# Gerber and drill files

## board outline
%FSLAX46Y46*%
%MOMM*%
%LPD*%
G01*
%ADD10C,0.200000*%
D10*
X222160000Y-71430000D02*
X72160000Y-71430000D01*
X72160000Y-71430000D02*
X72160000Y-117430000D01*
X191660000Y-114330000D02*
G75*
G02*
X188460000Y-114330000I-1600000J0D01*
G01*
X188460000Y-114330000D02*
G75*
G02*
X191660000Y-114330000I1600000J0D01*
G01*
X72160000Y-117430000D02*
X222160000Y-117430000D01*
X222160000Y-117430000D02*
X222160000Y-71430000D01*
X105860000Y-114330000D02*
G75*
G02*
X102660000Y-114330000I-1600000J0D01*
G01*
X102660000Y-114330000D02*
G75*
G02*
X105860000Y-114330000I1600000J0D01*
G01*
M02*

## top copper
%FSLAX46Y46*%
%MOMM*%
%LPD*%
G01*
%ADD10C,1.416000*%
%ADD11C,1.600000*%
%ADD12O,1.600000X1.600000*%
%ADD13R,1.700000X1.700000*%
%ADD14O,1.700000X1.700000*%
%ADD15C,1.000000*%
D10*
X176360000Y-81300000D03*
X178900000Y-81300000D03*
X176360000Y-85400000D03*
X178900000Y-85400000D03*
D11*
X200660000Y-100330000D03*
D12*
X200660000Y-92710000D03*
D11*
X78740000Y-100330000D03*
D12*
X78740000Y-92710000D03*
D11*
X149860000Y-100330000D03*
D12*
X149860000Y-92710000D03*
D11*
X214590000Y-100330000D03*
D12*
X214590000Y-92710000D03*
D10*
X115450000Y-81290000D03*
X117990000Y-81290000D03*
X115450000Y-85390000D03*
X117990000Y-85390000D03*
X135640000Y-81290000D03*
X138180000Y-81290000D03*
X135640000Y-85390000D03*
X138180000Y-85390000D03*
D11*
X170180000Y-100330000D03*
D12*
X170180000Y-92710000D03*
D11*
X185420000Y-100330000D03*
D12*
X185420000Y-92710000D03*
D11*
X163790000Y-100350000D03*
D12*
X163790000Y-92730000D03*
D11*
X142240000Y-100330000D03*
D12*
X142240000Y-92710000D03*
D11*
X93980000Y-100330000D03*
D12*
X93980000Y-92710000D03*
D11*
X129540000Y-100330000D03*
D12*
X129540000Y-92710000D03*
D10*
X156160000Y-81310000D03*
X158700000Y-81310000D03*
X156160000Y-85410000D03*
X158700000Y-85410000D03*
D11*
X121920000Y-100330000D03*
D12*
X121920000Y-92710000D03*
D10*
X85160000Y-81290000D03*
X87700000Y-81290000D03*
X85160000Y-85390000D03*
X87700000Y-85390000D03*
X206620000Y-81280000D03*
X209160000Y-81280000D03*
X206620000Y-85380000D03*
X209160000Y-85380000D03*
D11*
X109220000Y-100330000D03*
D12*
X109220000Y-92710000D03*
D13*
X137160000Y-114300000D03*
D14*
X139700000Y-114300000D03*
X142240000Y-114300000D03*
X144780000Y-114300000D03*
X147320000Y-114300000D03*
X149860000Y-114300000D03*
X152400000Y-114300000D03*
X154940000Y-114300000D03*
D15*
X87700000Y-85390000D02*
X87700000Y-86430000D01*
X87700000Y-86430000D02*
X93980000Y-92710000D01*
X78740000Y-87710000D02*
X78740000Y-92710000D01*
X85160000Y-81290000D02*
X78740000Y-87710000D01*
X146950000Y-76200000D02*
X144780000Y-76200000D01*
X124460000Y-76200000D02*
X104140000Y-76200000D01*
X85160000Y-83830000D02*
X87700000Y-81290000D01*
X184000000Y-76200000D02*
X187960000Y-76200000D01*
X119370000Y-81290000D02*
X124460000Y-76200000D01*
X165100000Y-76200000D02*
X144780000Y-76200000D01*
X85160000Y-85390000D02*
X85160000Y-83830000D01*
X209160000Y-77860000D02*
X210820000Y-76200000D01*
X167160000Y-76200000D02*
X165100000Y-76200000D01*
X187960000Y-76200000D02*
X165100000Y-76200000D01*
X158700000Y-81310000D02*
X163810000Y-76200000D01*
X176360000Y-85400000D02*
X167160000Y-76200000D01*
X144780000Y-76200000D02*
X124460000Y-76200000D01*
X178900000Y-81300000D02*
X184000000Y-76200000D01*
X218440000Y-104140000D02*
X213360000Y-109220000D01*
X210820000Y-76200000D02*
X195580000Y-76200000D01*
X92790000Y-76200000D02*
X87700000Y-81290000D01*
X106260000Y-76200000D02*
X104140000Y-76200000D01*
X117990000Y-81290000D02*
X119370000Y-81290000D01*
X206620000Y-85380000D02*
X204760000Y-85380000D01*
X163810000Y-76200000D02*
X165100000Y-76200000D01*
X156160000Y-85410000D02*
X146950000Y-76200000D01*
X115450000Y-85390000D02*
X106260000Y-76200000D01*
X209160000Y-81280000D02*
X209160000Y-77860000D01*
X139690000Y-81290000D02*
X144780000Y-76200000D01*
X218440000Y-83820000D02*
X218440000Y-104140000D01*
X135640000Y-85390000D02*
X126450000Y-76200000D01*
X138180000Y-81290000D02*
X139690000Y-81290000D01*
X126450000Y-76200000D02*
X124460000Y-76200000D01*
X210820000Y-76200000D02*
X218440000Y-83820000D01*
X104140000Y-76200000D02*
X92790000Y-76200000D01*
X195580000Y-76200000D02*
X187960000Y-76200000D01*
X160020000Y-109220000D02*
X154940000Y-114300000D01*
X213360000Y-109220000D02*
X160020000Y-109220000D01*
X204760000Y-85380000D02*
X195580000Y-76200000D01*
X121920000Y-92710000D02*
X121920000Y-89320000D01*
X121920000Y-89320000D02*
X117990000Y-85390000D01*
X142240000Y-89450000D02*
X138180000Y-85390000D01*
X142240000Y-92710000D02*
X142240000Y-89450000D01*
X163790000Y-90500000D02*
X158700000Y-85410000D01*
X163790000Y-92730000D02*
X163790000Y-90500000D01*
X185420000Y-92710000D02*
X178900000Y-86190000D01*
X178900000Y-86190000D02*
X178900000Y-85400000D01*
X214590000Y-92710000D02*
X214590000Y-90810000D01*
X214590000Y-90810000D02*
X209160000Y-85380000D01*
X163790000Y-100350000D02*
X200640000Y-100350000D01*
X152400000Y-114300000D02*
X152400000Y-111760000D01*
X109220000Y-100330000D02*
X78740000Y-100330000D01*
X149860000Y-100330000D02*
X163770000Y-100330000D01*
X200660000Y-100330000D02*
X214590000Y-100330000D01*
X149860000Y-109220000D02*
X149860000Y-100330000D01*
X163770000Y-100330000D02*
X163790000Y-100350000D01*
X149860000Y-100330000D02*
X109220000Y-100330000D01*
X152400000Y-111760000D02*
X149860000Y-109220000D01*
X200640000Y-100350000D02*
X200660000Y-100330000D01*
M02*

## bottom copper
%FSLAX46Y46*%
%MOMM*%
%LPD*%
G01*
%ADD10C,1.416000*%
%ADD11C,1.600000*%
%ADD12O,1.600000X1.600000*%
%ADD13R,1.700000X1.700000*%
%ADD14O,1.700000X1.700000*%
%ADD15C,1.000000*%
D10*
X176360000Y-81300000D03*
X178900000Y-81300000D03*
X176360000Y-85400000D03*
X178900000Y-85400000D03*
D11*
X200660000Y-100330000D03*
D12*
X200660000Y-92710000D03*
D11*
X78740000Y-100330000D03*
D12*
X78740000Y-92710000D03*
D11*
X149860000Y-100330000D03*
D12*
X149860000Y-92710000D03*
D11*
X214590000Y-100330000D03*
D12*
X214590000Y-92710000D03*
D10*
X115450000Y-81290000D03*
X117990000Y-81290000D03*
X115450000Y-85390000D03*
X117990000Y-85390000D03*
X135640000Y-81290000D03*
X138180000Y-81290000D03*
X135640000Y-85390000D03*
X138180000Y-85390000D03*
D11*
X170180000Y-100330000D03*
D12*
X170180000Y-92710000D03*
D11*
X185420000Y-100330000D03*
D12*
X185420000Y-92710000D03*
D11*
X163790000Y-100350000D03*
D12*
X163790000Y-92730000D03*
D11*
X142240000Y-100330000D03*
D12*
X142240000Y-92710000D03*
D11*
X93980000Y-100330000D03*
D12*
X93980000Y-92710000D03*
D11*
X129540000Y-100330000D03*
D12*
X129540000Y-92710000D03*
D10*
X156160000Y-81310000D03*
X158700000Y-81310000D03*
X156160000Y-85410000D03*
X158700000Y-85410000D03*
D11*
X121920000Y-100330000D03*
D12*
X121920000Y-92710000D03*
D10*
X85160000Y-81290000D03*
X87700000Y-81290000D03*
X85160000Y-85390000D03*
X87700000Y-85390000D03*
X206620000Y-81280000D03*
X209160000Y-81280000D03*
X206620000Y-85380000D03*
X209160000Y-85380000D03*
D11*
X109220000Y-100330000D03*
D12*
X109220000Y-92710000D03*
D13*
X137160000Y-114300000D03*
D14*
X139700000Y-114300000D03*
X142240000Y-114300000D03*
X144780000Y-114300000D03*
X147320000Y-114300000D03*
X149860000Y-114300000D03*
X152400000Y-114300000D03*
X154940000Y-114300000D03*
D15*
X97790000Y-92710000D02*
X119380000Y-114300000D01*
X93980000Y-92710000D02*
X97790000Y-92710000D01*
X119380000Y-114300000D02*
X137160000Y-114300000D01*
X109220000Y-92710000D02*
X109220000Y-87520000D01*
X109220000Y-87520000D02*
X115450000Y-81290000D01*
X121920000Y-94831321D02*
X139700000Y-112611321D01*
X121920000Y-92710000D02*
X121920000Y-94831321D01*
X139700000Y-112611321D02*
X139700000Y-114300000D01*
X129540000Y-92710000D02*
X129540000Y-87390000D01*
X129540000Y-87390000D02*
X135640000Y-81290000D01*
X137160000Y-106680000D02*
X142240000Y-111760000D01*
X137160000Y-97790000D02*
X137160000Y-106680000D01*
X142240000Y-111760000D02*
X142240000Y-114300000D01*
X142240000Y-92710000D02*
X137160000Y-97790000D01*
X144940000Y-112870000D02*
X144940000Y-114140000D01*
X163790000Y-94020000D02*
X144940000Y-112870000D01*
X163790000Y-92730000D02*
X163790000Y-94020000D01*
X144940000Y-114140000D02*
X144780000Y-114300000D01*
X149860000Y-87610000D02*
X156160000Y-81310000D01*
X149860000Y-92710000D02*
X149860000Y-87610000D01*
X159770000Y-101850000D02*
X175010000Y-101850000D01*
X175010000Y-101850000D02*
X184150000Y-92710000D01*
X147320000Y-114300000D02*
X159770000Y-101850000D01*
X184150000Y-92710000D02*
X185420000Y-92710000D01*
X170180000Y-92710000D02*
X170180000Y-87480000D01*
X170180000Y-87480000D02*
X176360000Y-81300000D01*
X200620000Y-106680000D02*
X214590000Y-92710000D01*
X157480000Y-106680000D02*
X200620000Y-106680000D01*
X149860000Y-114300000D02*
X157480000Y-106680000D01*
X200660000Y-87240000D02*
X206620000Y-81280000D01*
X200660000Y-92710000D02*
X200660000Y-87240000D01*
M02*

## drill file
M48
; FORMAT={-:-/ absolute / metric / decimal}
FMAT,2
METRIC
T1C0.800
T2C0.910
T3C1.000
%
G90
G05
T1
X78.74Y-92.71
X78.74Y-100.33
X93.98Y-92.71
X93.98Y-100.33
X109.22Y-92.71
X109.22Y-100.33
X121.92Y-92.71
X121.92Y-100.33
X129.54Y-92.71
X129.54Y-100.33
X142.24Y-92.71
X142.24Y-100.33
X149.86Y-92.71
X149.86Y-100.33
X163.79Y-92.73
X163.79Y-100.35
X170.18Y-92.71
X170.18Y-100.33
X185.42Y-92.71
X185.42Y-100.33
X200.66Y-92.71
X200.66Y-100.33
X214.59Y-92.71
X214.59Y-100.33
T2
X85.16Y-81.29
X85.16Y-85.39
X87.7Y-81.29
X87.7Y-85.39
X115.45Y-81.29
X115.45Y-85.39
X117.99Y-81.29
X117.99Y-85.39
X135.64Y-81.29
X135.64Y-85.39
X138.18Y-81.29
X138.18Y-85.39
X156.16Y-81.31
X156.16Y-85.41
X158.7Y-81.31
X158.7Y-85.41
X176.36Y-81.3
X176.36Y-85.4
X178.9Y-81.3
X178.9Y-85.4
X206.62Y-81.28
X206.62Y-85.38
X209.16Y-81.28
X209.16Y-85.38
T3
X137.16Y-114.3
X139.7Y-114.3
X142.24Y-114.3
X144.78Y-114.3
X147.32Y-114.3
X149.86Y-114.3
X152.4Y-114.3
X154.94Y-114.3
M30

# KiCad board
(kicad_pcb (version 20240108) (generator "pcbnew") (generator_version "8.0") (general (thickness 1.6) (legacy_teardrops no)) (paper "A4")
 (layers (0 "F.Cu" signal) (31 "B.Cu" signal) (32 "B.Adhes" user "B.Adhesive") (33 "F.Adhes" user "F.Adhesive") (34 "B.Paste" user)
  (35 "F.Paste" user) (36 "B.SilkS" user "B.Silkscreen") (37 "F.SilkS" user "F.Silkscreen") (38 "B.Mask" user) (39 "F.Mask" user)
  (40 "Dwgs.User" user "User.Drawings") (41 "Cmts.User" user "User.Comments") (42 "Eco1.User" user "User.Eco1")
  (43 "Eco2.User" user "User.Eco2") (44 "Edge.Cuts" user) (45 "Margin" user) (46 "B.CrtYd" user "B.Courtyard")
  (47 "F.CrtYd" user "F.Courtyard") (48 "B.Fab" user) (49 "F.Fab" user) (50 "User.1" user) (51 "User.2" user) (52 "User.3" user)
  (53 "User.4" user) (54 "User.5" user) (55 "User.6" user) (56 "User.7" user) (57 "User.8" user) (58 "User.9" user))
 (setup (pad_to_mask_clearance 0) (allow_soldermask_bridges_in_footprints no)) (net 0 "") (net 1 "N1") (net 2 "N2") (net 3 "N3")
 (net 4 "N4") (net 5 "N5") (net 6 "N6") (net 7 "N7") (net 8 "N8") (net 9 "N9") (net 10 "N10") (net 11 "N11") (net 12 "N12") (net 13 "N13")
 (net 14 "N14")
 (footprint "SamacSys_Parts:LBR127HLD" (layer "F.Cu") (at 176.36 81.3 90)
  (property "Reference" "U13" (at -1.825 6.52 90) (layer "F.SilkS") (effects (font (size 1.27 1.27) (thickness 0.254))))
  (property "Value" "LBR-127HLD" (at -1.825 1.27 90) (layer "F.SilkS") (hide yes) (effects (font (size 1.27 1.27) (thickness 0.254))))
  (pad "1" thru_hole circle (at 0 0 90) (size 1.416 1.416) (drill 0.91) (layers "*.Cu" "*.Mask") (remove_unused_layers no) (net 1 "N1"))
  (pad "2" thru_hole circle (at 0 2.54 90) (size 1.416 1.416) (drill 0.91) (layers "*.Cu" "*.Mask") (remove_unused_layers no) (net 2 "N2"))
  (pad "3" thru_hole circle (at -4.1 0 90) (size 1.416 1.416) (drill 0.91) (layers "*.Cu" "*.Mask") (remove_unused_layers no) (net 2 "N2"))
  (pad "4" thru_hole circle (at -4.1 2.54 90) (size 1.416 1.416) (drill 0.91) (layers "*.Cu" "*.Mask") (remove_unused_layers no)
   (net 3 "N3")))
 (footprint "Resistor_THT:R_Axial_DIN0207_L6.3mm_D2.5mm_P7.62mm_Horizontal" (layer "F.Cu") (at 200.66 100.33 90)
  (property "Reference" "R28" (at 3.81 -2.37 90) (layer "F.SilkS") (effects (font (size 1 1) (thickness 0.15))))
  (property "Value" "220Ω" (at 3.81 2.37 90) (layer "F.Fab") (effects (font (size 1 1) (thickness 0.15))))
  (pad "1" thru_hole circle (at 0 0 90) (size 1.6 1.6) (drill 0.8) (layers "*.Cu" "*.Mask") (remove_unused_layers no) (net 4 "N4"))
  (pad "2" thru_hole oval (at 7.62 0 90) (size 1.6 1.6) (drill 0.8) (layers "*.Cu" "*.Mask") (remove_unused_layers no) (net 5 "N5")))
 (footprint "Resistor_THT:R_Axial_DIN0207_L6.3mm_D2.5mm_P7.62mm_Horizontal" (layer "F.Cu") (at 78.74 100.33 90)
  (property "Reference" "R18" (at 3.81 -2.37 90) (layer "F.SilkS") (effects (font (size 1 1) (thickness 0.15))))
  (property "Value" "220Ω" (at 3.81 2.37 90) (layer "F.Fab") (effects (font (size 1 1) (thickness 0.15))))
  (pad "1" thru_hole circle (at 0 0 90) (size 1.6 1.6) (drill 0.8) (layers "*.Cu" "*.Mask") (remove_unused_layers no) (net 4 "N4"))
  (pad "2" thru_hole oval (at 7.62 0 90) (size 1.6 1.6) (drill 0.8) (layers "*.Cu" "*.Mask") (remove_unused_layers no) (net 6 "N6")))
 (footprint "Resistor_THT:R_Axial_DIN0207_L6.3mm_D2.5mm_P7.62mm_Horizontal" (layer "F.Cu") (at 149.86 100.33 90)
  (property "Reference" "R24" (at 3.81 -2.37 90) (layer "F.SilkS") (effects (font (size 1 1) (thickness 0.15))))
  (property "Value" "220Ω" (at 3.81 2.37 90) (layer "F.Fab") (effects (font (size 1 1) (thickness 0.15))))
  (pad "1" thru_hole circle (at 0 0 90) (size 1.6 1.6) (drill 0.8) (layers "*.Cu" "*.Mask") (remove_unused_layers no) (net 4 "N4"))
  (pad "2" thru_hole oval (at 7.62 0 90) (size 1.6 1.6) (drill 0.8) (layers "*.Cu" "*.Mask") (remove_unused_layers no) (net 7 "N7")))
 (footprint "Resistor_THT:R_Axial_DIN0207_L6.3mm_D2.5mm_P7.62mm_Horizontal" (layer "F.Cu") (at 214.59 100.33 90)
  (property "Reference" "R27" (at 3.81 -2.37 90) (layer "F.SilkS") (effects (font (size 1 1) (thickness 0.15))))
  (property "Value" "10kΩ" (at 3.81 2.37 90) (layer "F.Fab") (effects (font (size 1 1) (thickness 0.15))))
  (pad "1" thru_hole circle (at 0 0 90) (size 1.6 1.6) (drill 0.8) (layers "*.Cu" "*.Mask") (remove_unused_layers no) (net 4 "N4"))
  (pad "2" thru_hole oval (at 7.62 0 90) (size 1.6 1.6) (drill 0.8) (layers "*.Cu" "*.Mask") (remove_unused_layers no) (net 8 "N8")))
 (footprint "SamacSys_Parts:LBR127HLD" (layer "F.Cu") (at 115.45 81.29 90)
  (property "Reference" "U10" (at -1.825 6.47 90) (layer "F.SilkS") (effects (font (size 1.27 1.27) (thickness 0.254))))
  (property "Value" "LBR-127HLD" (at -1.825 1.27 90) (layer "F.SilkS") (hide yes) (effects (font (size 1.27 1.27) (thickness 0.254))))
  (pad "1" thru_hole circle (at 0 0 90) (size 1.416 1.416) (drill 0.91) (layers "*.Cu" "*.Mask") (remove_unused_layers no) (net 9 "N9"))
  (pad "2" thru_hole circle (at 0 2.54 90) (size 1.416 1.416) (drill 0.91) (layers "*.Cu" "*.Mask") (remove_unused_layers no) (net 2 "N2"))
  (pad "3" thru_hole circle (at -4.1 0 90) (size 1.416 1.416) (drill 0.91) (layers "*.Cu" "*.Mask") (remove_unused_layers no) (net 2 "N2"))
  (pad "4" thru_hole circle (at -4.1 2.54 90) (size 1.416 1.416) (drill 0.91) (layers "*.Cu" "*.Mask") (remove_unused_layers no)
   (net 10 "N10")))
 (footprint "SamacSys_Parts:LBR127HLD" (layer "F.Cu") (at 135.64 81.29 90)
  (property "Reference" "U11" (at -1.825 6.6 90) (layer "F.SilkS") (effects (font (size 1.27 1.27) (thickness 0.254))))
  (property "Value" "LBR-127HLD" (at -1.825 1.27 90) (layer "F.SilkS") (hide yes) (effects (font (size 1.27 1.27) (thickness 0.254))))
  (pad "1" thru_hole circle (at 0 0 90) (size 1.416 1.416) (drill 0.91) (layers "*.Cu" "*.Mask") (remove_unused_layers no) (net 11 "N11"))
  (pad "2" thru_hole circle (at 0 2.54 90) (size 1.416 1.416) (drill 0.91) (layers "*.Cu" "*.Mask") (remove_unused_layers no) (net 2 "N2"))
  (pad "3" thru_hole circle (at -4.1 0 90) (size 1.416 1.416) (drill 0.91) (layers "*.Cu" "*.Mask") (remove_unused_layers no) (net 2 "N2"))
  (pad "4" thru_hole circle (at -4.1 2.54 90) (size 1.416 1.416) (drill 0.91) (layers "*.Cu" "*.Mask") (remove_unused_layers no)
   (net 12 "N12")))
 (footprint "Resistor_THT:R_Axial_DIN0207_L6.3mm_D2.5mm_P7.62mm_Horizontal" (layer "F.Cu") (at 170.18 100.33 90)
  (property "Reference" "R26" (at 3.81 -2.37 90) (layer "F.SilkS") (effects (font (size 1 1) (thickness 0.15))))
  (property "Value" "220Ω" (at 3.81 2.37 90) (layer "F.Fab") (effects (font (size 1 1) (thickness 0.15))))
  (pad "1" thru_hole circle (at 0 0 90) (size 1.6 1.6) (drill 0.8) (layers "*.Cu" "*.Mask") (remove_unused_layers no) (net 4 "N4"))
  (pad "2" thru_hole oval (at 7.62 0 90) (size 1.6 1.6) (drill 0.8) (layers "*.Cu" "*.Mask") (remove_unused_layers no) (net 1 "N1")))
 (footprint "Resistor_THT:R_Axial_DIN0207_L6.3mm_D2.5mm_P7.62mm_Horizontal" (layer "F.Cu") (at 185.42 100.33 90)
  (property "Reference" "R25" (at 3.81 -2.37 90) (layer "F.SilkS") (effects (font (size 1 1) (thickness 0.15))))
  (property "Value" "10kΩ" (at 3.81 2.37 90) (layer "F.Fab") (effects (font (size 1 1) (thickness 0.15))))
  (pad "1" thru_hole circle (at 0 0 90) (size 1.6 1.6) (drill 0.8) (layers "*.Cu" "*.Mask") (remove_unused_layers no) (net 4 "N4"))
  (pad "2" thru_hole oval (at 7.62 0 90) (size 1.6 1.6) (drill 0.8) (layers "*.Cu" "*.Mask") (remove_unused_layers no) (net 3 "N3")))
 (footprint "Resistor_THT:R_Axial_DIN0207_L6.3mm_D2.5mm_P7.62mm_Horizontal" (layer "F.Cu") (at 163.79 100.35 90)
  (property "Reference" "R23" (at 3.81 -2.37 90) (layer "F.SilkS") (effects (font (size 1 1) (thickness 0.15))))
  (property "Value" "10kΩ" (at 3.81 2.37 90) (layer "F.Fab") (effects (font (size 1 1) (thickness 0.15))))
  (pad "1" thru_hole circle (at 0 0 90) (size 1.6 1.6) (drill 0.8) (layers "*.Cu" "*.Mask") (remove_unused_layers no) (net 4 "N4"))
  (pad "2" thru_hole oval (at 7.62 0 90) (size 1.6 1.6) (drill 0.8) (layers "*.Cu" "*.Mask") (remove_unused_layers no) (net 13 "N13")))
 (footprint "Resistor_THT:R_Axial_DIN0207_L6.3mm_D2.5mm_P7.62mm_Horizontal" (layer "F.Cu") (at 142.24 100.33 90)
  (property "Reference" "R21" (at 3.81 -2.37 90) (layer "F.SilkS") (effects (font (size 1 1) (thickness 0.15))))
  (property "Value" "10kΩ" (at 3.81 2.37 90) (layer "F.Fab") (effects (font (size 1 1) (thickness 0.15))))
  (pad "1" thru_hole circle (at 0 0 90) (size 1.6 1.6) (drill 0.8) (layers "*.Cu" "*.Mask") (remove_unused_layers no) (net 4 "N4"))
  (pad "2" thru_hole oval (at 7.62 0 90) (size 1.6 1.6) (drill 0.8) (layers "*.Cu" "*.Mask") (remove_unused_layers no) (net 12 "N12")))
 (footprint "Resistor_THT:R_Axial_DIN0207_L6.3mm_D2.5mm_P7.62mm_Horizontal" (layer "F.Cu") (at 93.98 100.33 90)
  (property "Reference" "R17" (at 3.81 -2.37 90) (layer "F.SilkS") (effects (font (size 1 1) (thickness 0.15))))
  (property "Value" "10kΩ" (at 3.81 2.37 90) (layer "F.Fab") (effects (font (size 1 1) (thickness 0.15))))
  (pad "1" thru_hole circle (at 0 0 90) (size 1.6 1.6) (drill 0.8) (layers "*.Cu" "*.Mask") (remove_unused_layers no) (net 4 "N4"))
  (pad "2" thru_hole oval (at 7.62 0 90) (size 1.6 1.6) (drill 0.8) (layers "*.Cu" "*.Mask") (remove_unused_layers no) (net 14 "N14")))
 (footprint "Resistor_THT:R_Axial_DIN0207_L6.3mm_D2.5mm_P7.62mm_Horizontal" (layer "F.Cu") (at 129.54 100.33 90)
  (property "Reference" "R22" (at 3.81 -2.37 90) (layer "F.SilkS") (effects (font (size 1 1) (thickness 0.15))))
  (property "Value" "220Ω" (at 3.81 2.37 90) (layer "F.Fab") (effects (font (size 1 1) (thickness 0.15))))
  (pad "1" thru_hole circle (at 0 0 90) (size 1.6 1.6) (drill 0.8) (layers "*.Cu" "*.Mask") (remove_unused_layers no) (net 4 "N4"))
  (pad "2" thru_hole oval (at 7.62 0 90) (size 1.6 1.6) (drill 0.8) (layers "*.Cu" "*.Mask") (remove_unused_layers no) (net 11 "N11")))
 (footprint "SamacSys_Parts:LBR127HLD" (layer "F.Cu") (at 156.16 81.31 90)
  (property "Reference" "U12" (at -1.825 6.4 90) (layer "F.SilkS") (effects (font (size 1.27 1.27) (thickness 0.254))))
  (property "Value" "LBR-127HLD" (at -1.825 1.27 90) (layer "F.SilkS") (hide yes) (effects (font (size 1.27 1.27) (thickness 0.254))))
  (pad "1" thru_hole circle (at 0 0 90) (size 1.416 1.416) (drill 0.91) (layers "*.Cu" "*.Mask") (remove_unused_layers no) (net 7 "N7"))
  (pad "2" thru_hole circle (at 0 2.54 90) (size 1.416 1.416) (drill 0.91) (layers "*.Cu" "*.Mask") (remove_unused_layers no) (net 2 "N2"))
  (pad "3" thru_hole circle (at -4.1 0 90) (size 1.416 1.416) (drill 0.91) (layers "*.Cu" "*.Mask") (remove_unused_layers no) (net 2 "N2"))
  (pad "4" thru_hole circle (at -4.1 2.54 90) (size 1.416 1.416) (drill 0.91) (layers "*.Cu" "*.Mask") (remove_unused_layers no)
   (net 13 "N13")))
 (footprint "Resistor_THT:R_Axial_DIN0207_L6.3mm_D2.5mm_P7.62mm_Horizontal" (layer "F.Cu") (at 121.92 100.33 90)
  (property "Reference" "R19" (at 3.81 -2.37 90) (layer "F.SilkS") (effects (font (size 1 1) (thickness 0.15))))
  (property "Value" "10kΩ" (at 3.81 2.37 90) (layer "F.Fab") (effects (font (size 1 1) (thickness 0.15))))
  (pad "1" thru_hole circle (at 0 0 90) (size 1.6 1.6) (drill 0.8) (layers "*.Cu" "*.Mask") (remove_unused_layers no) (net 4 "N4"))
  (pad "2" thru_hole oval (at 7.62 0 90) (size 1.6 1.6) (drill 0.8) (layers "*.Cu" "*.Mask") (remove_unused_layers no) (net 10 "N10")))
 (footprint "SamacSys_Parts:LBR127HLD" (layer "F.Cu") (at 85.16 81.29 90)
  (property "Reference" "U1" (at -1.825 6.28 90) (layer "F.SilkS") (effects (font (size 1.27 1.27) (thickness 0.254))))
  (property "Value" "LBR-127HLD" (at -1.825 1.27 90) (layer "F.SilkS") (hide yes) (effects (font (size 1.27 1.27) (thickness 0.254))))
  (pad "1" thru_hole circle (at 0 0 90) (size 1.416 1.416) (drill 0.91) (layers "*.Cu" "*.Mask") (remove_unused_layers no) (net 6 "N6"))
  (pad "2" thru_hole circle (at 0 2.54 90) (size 1.416 1.416) (drill 0.91) (layers "*.Cu" "*.Mask") (remove_unused_layers no) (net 2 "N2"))
  (pad "3" thru_hole circle (at -4.1 0 90) (size 1.416 1.416) (drill 0.91) (layers "*.Cu" "*.Mask") (remove_unused_layers no) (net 2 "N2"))
  (pad "4" thru_hole circle (at -4.1 2.54 90) (size 1.416 1.416) (drill 0.91) (layers "*.Cu" "*.Mask") (remove_unused_layers no)
   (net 14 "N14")))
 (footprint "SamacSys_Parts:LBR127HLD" (layer "F.Cu") (at 206.62 81.28 90)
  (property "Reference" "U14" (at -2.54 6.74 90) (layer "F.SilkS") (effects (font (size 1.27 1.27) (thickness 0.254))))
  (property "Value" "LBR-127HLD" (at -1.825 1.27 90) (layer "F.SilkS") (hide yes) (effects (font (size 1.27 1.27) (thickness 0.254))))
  (pad "1" thru_hole circle (at 0 0 90) (size 1.416 1.416) (drill 0.91) (layers "*.Cu" "*.Mask") (remove_unused_layers no) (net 5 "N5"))
  (pad "2" thru_hole circle (at 0 2.54 90) (size 1.416 1.416) (drill 0.91) (layers "*.Cu" "*.Mask") (remove_unused_layers no) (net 2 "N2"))
  (pad "3" thru_hole circle (at -4.1 0 90) (size 1.416 1.416) (drill 0.91) (layers "*.Cu" "*.Mask") (remove_unused_layers no) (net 2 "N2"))
  (pad "4" thru_hole circle (at -4.1 2.54 90) (size 1.416 1.416) (drill 0.91) (layers "*.Cu" "*.Mask") (remove_unused_layers no)
   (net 8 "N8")))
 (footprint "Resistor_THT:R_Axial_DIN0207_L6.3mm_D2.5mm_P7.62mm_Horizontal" (layer "F.Cu") (at 109.22 100.33 90)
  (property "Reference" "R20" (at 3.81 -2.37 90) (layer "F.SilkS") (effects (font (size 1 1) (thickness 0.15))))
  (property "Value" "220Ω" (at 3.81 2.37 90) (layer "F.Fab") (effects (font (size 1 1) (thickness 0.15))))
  (pad "1" thru_hole circle (at 0 0 90) (size 1.6 1.6) (drill 0.8) (layers "*.Cu" "*.Mask") (remove_unused_layers no) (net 4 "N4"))
  (pad "2" thru_hole oval (at 7.62 0 90) (size 1.6 1.6) (drill 0.8) (layers "*.Cu" "*.Mask") (remove_unused_layers no) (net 9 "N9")))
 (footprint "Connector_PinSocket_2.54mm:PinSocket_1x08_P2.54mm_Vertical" (layer "F.Cu") (at 137.16 114.3 90)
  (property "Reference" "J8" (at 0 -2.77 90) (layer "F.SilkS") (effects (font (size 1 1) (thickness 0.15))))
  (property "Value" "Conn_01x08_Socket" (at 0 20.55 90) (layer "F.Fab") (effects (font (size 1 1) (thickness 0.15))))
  (pad "1" thru_hole rect (at 0 0 90) (size 1.7 1.7) (drill 1) (layers "*.Cu" "*.Mask") (remove_unused_layers no) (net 14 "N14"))
  (pad "2" thru_hole oval (at 0 2.54 90) (size 1.7 1.7) (drill 1) (layers "*.Cu" "*.Mask") (remove_unused_layers no) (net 10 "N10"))
  (pad "3" thru_hole oval (at 0 5.08 90) (size 1.7 1.7) (drill 1) (layers "*.Cu" "*.Mask") (remove_unused_layers no) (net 12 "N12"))
  (pad "4" thru_hole oval (at 0 7.62 90) (size 1.7 1.7) (drill 1) (layers "*.Cu" "*.Mask") (remove_unused_layers no) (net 13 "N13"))
  (pad "5" thru_hole oval (at 0 10.16 90) (size 1.7 1.7) (drill 1) (layers "*.Cu" "*.Mask") (remove_unused_layers no) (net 3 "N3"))
  (pad "6" thru_hole oval (at 0 12.7 90) (size 1.7 1.7) (drill 1) (layers "*.Cu" "*.Mask") (remove_unused_layers no) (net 8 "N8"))
  (pad "7" thru_hole oval (at 0 15.24 90) (size 1.7 1.7) (drill 1) (layers "*.Cu" "*.Mask") (remove_unused_layers no) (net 4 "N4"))
  (pad "8" thru_hole oval (at 0 17.78 90) (size 1.7 1.7) (drill 1) (layers "*.Cu" "*.Mask") (remove_unused_layers no) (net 2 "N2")))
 (gr_line (start 222.16 71.43) (end 72.16 71.43) (stroke (width 0.2) (type default)) (layer "Edge.Cuts"))
 (gr_line (start 72.16 71.43) (end 72.16 117.43) (stroke (width 0.2) (type default)) (layer "Edge.Cuts"))
 (gr_circle (center 190.06 114.33) (end 191.66 114.33) (stroke (width 0.2) (type default)) (fill none) (layer "Edge.Cuts"))
 (gr_line (start 72.16 117.43) (end 222.16 117.43) (stroke (width 0.2) (type default)) (layer "Edge.Cuts"))
 (gr_line (start 222.16 117.43) (end 222.16 71.43) (stroke (width 0.2) (type default)) (layer "Edge.Cuts"))
 (gr_circle (center 104.26 114.33) (end 105.86 114.33) (stroke (width 0.2) (type default)) (fill none) (layer "Edge.Cuts"))
 (segment (start 87.7 85.39) (end 87.7 86.43) (width 1) (layer "F.Cu") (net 14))
 (segment (start 87.7 86.43) (end 93.98 92.71) (width 1) (layer "F.Cu") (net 14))
 (segment (start 97.79 92.71) (end 119.38 114.3) (width 1) (layer "B.Cu") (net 14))
 (segment (start 93.98 92.71) (end 97.79 92.71) (width 1) (layer "B.Cu") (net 14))
 (segment (start 119.38 114.3) (end 137.16 114.3) (width 1) (layer "B.Cu") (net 14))
 (segment (start 78.74 87.71) (end 78.74 92.71) (width 1) (layer "F.Cu") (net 6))
 (segment (start 85.16 81.29) (end 78.74 87.71) (width 1) (layer "F.Cu") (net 6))
 (segment (start 146.95 76.2) (end 144.78 76.2) (width 1) (layer "F.Cu") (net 2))
 (segment (start 124.46 76.2) (end 104.14 76.2) (width 1) (layer "F.Cu") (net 2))
 (segment (start 85.16 83.83) (end 87.7 81.29) (width 1) (layer "F.Cu") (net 2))
 (segment (start 184 76.2) (end 187.96 76.2) (width 1) (layer "F.Cu") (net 2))
 (segment (start 119.37 81.29) (end 124.46 76.2) (width 1) (layer "F.Cu") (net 2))
 (segment (start 165.1 76.2) (end 144.78 76.2) (width 1) (layer "F.Cu") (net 2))
 (segment (start 85.16 85.39) (end 85.16 83.83) (width 1) (layer "F.Cu") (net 2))
 (segment (start 209.16 77.86) (end 210.82 76.2) (width 1) (layer "F.Cu") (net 2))
 (segment (start 167.16 76.2) (end 165.1 76.2) (width 1) (layer "F.Cu") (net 2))
 (segment (start 187.96 76.2) (end 165.1 76.2) (width 1) (layer "F.Cu") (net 2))
 (segment (start 158.7 81.31) (end 163.81 76.2) (width 1) (layer "F.Cu") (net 2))
 (segment (start 176.36 85.4) (end 167.16 76.2) (width 1) (layer "F.Cu") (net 2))
 (segment (start 144.78 76.2) (end 124.46 76.2) (width 1) (layer "F.Cu") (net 2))
 (segment (start 178.9 81.3) (end 184 76.2) (width 1) (layer "F.Cu") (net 2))
 (segment (start 218.44 104.14) (end 213.36 109.22) (width 1) (layer "F.Cu") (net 2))
 (segment (start 210.82 76.2) (end 195.58 76.2) (width 1) (layer "F.Cu") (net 2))
 (segment (start 92.79 76.2) (end 87.7 81.29) (width 1) (layer "F.Cu") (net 2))
 (segment (start 106.26 76.2) (end 104.14 76.2) (width 1) (layer "F.Cu") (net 2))
 (segment (start 117.99 81.29) (end 119.37 81.29) (width 1) (layer "F.Cu") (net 2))
 (segment (start 206.62 85.38) (end 204.76 85.38) (width 1) (layer "F.Cu") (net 2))
 (segment (start 163.81 76.2) (end 165.1 76.2) (width 1) (layer "F.Cu") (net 2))
 (segment (start 156.16 85.41) (end 146.95 76.2) (width 1) (layer "F.Cu") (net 2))
 (segment (start 115.45 85.39) (end 106.26 76.2) (width 1) (layer "F.Cu") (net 2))
 (segment (start 209.16 81.28) (end 209.16 77.86) (width 1) (layer "F.Cu") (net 2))
 (segment (start 139.69 81.29) (end 144.78 76.2) (width 1) (layer "F.Cu") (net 2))
 (segment (start 218.44 83.82) (end 218.44 104.14) (width 1) (layer "F.Cu") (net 2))
 (segment (start 135.64 85.39) (end 126.45 76.2) (width 1) (layer "F.Cu") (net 2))
 (segment (start 138.18 81.29) (end 139.69 81.29) (width 1) (layer "F.Cu") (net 2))
 (segment (start 126.45 76.2) (end 124.46 76.2) (width 1) (layer "F.Cu") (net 2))
 (segment (start 210.82 76.2) (end 218.44 83.82) (width 1) (layer "F.Cu") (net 2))
 (segment (start 104.14 76.2) (end 92.79 76.2) (width 1) (layer "F.Cu") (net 2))
 (segment (start 195.58 76.2) (end 187.96 76.2) (width 1) (layer "F.Cu") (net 2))
 (segment (start 160.02 109.22) (end 154.94 114.3) (width 1) (layer "F.Cu") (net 2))
 (segment (start 213.36 109.22) (end 160.02 109.22) (width 1) (layer "F.Cu") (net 2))
 (segment (start 204.76 85.38) (end 195.58 76.2) (width 1) (layer "F.Cu") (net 2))
 (segment (start 109.22 92.71) (end 109.22 87.52) (width 1) (layer "B.Cu") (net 9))
 (segment (start 109.22 87.52) (end 115.45 81.29) (width 1) (layer "B.Cu") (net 9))
 (segment (start 121.92 92.71) (end 121.92 89.32) (width 1) (layer "F.Cu") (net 10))
 (segment (start 121.92 89.32) (end 117.99 85.39) (width 1) (layer "F.Cu") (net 10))
 (segment (start 121.92 94.831321) (end 139.7 112.611321) (width 1) (layer "B.Cu") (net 10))
 (segment (start 121.92 92.71) (end 121.92 94.831321) (width 1) (layer "B.Cu") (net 10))
 (segment (start 139.7 112.611321) (end 139.7 114.3) (width 1) (layer "B.Cu") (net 10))
 (segment (start 129.54 92.71) (end 129.54 87.39) (width 1) (layer "B.Cu") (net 11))
 (segment (start 129.54 87.39) (end 135.64 81.29) (width 1) (layer "B.Cu") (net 11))
 (segment (start 142.24 89.45) (end 138.18 85.39) (width 1) (layer "F.Cu") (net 12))
 (segment (start 142.24 92.71) (end 142.24 89.45) (width 1) (layer "F.Cu") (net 12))
 (segment (start 137.16 106.68) (end 142.24 111.76) (width 1) (layer "B.Cu") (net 12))
 (segment (start 137.16 97.79) (end 137.16 106.68) (width 1) (layer "B.Cu") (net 12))
 (segment (start 142.24 111.76) (end 142.24 114.3) (width 1) (layer "B.Cu") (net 12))
 (segment (start 142.24 92.71) (end 137.16 97.79) (width 1) (layer "B.Cu") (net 12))
 (segment (start 163.79 90.5) (end 158.7 85.41) (width 1) (layer "F.Cu") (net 13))
 (segment (start 163.79 92.73) (end 163.79 90.5) (width 1) (layer "F.Cu") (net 13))
 (segment (start 144.94 112.87) (end 144.94 114.14) (width 1) (layer "B.Cu") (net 13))
 (segment (start 163.79 94.02) (end 144.94 112.87) (width 1) (layer "B.Cu") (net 13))
 (segment (start 163.79 92.73) (end 163.79 94.02) (width 1) (layer "B.Cu") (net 13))
 (segment (start 144.94 114.14) (end 144.78 114.3) (width 1) (layer "B.Cu") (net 13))
 (segment (start 149.86 87.61) (end 156.16 81.31) (width 1) (layer "B.Cu") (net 7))
 (segment (start 149.86 92.71) (end 149.86 87.61) (width 1) (layer "B.Cu") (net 7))
 (segment (start 185.42 92.71) (end 178.9 86.19) (width 1) (layer "F.Cu") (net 3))
 (segment (start 178.9 86.19) (end 178.9 85.4) (width 1) (layer "F.Cu") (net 3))
 (segment (start 159.77 101.85) (end 175.01 101.85) (width 1) (layer "B.Cu") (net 3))
 (segment (start 175.01 101.85) (end 184.15 92.71) (width 1) (layer "B.Cu") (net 3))
 (segment (start 147.32 114.3) (end 159.77 101.85) (width 1) (layer "B.Cu") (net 3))
 (segment (start 184.15 92.71) (end 185.42 92.71) (width 1) (layer "B.Cu") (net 3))
 (segment (start 170.18 92.71) (end 170.18 87.48) (width 1) (layer "B.Cu") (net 1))
 (segment (start 170.18 87.48) (end 176.36 81.3) (width 1) (layer "B.Cu") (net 1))
 (segment (start 214.59 92.71) (end 214.59 90.81) (width 1) (layer "F.Cu") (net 8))
 (segment (start 214.59 90.81) (end 209.16 85.38) (width 1) (layer "F.Cu") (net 8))
 (segment (start 200.62 106.68) (end 214.59 92.71) (width 1) (layer "B.Cu") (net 8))
 (segment (start 157.48 106.68) (end 200.62 106.68) (width 1) (layer "B.Cu") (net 8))
 (segment (start 149.86 114.3) (end 157.48 106.68) (width 1) (layer "B.Cu") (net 8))
 (segment (start 200.66 87.24) (end 206.62 81.28) (width 1) (layer "B.Cu") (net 5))
 (segment (start 200.66 92.71) (end 200.66 87.24) (width 1) (layer "B.Cu") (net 5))
 (segment (start 163.79 100.35) (end 200.64 100.35) (width 1) (layer "F.Cu") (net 4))
 (segment (start 152.4 114.3) (end 152.4 111.76) (width 1) (layer "F.Cu") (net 4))
 (segment (start 109.22 100.33) (end 78.74 100.33) (width 1) (layer "F.Cu") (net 4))
 (segment (start 149.86 100.33) (end 163.77 100.33) (width 1) (layer "F.Cu") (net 4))
 (segment (start 200.66 100.33) (end 214.59 100.33) (width 1) (layer "F.Cu") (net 4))
 (segment (start 149.86 109.22) (end 149.86 100.33) (width 1) (layer "F.Cu") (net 4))
 (segment (start 163.77 100.33) (end 163.79 100.35) (width 1) (layer "F.Cu") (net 4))
 (segment (start 149.86 100.33) (end 109.22 100.33) (width 1) (layer "F.Cu") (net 4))
 (segment (start 152.4 111.76) (end 149.86 109.22) (width 1) (layer "F.Cu") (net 4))
 (segment (start 200.64 100.35) (end 200.66 100.33) (width 1) (layer "F.Cu") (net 4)))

